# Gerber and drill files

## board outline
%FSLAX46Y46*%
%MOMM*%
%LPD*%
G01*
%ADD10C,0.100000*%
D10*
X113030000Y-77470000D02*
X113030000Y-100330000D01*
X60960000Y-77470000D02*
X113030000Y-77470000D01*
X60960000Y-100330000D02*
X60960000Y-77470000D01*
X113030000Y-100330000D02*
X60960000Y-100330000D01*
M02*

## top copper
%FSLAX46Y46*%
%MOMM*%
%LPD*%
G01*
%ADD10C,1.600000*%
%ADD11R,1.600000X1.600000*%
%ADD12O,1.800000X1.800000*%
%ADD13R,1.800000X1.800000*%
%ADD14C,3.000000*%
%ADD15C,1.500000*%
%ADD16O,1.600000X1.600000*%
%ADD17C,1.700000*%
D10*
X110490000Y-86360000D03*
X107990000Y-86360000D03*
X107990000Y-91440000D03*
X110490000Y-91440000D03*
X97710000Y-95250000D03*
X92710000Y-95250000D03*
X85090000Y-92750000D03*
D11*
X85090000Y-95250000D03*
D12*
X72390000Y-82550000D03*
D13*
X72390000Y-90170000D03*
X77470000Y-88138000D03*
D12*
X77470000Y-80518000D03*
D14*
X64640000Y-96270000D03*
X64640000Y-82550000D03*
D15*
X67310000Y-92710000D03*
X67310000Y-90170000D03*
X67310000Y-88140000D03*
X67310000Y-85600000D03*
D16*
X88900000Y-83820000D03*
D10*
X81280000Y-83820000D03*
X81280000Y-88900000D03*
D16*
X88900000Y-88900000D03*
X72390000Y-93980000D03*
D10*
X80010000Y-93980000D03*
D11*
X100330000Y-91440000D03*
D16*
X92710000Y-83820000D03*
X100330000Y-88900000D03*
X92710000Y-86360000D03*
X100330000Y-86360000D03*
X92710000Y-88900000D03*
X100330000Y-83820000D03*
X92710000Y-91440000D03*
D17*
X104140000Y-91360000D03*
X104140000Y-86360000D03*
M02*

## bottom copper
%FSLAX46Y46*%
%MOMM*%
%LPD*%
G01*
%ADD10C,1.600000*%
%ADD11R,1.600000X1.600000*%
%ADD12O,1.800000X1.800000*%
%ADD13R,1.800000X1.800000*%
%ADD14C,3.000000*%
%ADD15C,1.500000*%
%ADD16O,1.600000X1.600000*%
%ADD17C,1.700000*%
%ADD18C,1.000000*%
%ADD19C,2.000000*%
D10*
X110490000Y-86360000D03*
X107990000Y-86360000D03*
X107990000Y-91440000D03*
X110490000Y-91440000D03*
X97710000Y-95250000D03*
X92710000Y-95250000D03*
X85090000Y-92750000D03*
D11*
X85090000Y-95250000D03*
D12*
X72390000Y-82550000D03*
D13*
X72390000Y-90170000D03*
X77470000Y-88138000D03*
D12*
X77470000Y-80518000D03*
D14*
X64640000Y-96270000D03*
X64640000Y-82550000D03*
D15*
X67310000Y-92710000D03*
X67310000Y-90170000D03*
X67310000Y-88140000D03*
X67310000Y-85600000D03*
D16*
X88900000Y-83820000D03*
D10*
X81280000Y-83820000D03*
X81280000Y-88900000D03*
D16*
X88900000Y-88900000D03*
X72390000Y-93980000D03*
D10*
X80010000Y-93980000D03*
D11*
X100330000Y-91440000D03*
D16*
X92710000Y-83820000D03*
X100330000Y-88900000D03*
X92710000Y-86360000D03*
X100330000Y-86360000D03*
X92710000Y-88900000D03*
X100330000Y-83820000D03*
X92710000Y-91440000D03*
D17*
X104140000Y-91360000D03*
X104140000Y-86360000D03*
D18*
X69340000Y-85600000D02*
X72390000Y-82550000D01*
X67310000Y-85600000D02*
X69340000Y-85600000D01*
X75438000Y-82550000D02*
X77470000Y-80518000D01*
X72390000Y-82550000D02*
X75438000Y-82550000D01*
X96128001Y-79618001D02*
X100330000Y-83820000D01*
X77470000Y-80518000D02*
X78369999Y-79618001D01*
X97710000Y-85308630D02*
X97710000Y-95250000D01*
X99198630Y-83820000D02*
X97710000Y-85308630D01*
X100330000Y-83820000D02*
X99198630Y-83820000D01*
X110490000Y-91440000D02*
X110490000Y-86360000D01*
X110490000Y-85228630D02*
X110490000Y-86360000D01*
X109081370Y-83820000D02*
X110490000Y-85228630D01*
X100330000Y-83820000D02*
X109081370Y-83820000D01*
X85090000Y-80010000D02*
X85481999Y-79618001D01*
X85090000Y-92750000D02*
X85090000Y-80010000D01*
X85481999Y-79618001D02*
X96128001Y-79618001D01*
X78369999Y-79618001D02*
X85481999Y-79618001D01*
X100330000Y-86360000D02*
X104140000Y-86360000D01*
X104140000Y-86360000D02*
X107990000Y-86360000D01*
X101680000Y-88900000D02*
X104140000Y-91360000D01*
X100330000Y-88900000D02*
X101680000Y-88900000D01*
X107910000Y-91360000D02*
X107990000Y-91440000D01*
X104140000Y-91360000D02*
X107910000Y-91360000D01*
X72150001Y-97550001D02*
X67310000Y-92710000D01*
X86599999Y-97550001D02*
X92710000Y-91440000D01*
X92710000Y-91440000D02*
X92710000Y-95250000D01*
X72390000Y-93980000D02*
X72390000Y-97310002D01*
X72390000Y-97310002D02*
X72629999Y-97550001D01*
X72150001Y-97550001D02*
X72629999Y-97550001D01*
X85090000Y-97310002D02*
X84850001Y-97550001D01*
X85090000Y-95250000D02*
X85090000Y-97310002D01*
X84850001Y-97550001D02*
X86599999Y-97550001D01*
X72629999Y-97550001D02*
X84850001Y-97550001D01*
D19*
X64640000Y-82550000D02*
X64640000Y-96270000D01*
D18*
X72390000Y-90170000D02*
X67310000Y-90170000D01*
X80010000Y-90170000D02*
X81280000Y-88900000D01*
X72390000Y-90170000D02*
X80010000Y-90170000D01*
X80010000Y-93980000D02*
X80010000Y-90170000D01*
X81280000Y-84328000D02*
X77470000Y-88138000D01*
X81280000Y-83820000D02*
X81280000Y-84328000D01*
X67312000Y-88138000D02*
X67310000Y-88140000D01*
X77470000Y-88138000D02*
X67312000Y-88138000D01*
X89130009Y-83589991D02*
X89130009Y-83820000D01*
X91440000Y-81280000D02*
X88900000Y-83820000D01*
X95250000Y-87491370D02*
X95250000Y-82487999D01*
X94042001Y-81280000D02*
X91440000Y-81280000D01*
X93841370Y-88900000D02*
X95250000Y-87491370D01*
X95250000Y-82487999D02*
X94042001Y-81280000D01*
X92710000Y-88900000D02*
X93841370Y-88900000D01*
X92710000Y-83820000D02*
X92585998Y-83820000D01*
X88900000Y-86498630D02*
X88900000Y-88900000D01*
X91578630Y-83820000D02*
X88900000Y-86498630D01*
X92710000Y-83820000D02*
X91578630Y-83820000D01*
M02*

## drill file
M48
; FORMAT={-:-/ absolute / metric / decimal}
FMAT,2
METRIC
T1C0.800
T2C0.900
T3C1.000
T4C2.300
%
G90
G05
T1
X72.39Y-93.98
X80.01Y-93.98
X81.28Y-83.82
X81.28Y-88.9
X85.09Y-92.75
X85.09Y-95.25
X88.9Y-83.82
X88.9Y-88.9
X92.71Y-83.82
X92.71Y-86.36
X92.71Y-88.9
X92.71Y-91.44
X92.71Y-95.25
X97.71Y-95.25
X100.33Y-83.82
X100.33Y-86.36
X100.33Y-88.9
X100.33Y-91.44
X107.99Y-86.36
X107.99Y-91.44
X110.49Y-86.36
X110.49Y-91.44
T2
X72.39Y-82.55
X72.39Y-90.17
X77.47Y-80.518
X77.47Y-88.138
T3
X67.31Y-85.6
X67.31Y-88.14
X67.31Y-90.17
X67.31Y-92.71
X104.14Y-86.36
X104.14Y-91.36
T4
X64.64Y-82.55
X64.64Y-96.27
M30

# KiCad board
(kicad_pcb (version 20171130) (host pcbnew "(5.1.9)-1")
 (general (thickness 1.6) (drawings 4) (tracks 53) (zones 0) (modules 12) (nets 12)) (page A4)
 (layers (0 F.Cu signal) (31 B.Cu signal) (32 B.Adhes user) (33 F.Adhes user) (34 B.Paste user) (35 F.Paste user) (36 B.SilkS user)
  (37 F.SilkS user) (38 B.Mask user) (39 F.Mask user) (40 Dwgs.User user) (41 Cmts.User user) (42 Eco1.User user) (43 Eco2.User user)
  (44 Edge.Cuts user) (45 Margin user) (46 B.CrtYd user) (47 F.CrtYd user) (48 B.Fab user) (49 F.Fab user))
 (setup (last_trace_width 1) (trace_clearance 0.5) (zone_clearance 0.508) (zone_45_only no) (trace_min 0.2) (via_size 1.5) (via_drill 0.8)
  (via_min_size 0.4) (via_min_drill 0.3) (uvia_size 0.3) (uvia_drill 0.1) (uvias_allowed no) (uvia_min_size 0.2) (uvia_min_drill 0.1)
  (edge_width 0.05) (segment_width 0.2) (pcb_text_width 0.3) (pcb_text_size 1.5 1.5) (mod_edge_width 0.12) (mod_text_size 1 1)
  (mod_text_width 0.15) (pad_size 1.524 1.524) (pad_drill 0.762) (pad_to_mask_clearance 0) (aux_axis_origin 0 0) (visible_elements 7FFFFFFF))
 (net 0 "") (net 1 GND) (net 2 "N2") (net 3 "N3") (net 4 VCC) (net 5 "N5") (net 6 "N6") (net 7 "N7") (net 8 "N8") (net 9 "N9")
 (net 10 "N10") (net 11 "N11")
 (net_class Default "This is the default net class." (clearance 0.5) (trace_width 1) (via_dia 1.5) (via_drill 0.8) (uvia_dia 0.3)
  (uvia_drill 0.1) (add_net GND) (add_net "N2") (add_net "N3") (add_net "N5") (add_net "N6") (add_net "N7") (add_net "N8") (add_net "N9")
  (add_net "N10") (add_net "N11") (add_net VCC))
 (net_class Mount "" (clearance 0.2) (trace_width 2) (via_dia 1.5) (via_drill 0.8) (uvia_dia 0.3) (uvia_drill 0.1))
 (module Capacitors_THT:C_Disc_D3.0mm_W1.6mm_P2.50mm (layer F.Cu) (at 110.49 86.36 180)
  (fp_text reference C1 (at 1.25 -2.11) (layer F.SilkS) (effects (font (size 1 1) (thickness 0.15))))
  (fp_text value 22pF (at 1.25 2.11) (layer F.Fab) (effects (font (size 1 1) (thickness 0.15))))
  (pad 1 thru_hole circle (at 0 0 180) (size 1.6 1.6) (drill 0.8) (layers *.Cu *.Mask) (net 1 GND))
  (pad 2 thru_hole circle (at 2.5 0 180) (size 1.6 1.6) (drill 0.8) (layers *.Cu *.Mask) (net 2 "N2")))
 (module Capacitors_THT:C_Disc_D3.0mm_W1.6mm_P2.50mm (layer F.Cu) (at 110.49 91.44 180)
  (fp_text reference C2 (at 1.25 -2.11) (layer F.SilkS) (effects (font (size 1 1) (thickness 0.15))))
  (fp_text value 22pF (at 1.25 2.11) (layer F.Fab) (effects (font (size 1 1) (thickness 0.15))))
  (pad 2 thru_hole circle (at 2.5 0 180) (size 1.6 1.6) (drill 0.8) (layers *.Cu *.Mask) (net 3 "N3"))
  (pad 1 thru_hole circle (at 0 0 180) (size 1.6 1.6) (drill 0.8) (layers *.Cu *.Mask) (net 1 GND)))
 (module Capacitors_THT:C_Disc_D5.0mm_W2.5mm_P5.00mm (layer F.Cu) (at 92.71 95.25)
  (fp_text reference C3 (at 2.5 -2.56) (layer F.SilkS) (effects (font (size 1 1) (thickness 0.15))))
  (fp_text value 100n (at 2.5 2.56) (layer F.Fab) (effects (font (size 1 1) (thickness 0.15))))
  (pad 2 thru_hole circle (at 5 0) (size 1.6 1.6) (drill 0.8) (layers *.Cu *.Mask) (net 1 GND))
  (pad 1 thru_hole circle (at 0 0) (size 1.6 1.6) (drill 0.8) (layers *.Cu *.Mask) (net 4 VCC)))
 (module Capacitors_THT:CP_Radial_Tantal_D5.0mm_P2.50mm (layer F.Cu) (at 85.09 95.25 90)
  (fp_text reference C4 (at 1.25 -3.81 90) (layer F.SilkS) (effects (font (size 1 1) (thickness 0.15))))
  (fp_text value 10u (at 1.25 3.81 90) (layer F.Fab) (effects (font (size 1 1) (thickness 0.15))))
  (pad 2 thru_hole circle (at 2.5 0 90) (size 1.6 1.6) (drill 0.8) (layers *.Cu *.Mask) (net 1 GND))
  (pad 1 thru_hole rect (at 0 0 90) (size 1.6 1.6) (drill 0.8) (layers *.Cu *.Mask) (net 4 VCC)))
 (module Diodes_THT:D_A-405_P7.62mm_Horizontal (layer F.Cu) (at 72.39 90.17 90)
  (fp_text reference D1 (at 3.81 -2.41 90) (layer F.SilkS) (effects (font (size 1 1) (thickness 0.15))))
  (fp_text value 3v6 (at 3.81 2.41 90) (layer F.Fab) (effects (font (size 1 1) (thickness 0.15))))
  (pad 2 thru_hole oval (at 7.62 0 90) (size 1.8 1.8) (drill 0.9) (layers *.Cu *.Mask) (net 1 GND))
  (pad 1 thru_hole rect (at 0 0 90) (size 1.8 1.8) (drill 0.9) (layers *.Cu *.Mask) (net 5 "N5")))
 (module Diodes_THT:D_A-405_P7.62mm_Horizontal (layer F.Cu) (at 77.47 88.138 90)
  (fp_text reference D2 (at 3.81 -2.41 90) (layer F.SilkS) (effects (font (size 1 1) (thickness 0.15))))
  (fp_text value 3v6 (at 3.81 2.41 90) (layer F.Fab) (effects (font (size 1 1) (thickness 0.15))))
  (pad 1 thru_hole rect (at 0 0 90) (size 1.8 1.8) (drill 0.9) (layers *.Cu *.Mask) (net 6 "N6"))
  (pad 2 thru_hole oval (at 7.62 0 90) (size 1.8 1.8) (drill 0.9) (layers *.Cu *.Mask) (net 1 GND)))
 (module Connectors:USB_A (layer B.Cu) (at 67.31 92.71 90)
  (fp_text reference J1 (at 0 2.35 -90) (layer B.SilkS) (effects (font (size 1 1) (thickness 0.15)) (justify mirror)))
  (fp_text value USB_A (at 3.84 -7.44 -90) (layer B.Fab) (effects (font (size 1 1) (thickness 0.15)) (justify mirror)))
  (pad 5 thru_hole circle (at -3.56 -2.67 180) (size 3 3) (drill 2.3) (layers *.Cu *.Mask) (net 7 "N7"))
  (pad 5 thru_hole circle (at 10.16 -2.67 180) (size 3 3) (drill 2.3) (layers *.Cu *.Mask) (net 7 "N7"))
  (pad 1 thru_hole circle (at 0 0 180) (size 1.5 1.5) (drill 1) (layers *.Cu *.Mask) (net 4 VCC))
  (pad 2 thru_hole circle (at 2.54 0 180) (size 1.5 1.5) (drill 1) (layers *.Cu *.Mask) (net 5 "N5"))
  (pad 3 thru_hole circle (at 4.57 0 180) (size 1.5 1.5) (drill 1) (layers *.Cu *.Mask) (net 6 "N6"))
  (pad 4 thru_hole circle (at 7.11 0 180) (size 1.5 1.5) (drill 1) (layers *.Cu *.Mask) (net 1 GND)))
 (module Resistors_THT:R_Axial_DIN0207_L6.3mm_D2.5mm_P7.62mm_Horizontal (layer F.Cu) (at 81.28 83.82)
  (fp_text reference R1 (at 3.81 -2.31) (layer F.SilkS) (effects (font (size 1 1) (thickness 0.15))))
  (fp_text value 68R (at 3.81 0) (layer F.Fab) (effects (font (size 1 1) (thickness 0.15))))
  (pad 2 thru_hole oval (at 7.62 0) (size 1.6 1.6) (drill 0.8) (layers *.Cu *.Mask) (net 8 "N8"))
  (pad 1 thru_hole circle (at 0 0) (size 1.6 1.6) (drill 0.8) (layers *.Cu *.Mask) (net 6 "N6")))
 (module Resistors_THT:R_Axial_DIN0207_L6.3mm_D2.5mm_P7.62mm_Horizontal (layer F.Cu) (at 81.28 88.9)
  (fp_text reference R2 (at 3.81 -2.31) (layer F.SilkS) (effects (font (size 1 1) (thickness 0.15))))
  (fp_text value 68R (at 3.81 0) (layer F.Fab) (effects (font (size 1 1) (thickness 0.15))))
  (pad 1 thru_hole circle (at 0 0) (size 1.6 1.6) (drill 0.8) (layers *.Cu *.Mask) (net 5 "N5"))
  (pad 2 thru_hole oval (at 7.62 0) (size 1.6 1.6) (drill 0.8) (layers *.Cu *.Mask) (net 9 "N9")))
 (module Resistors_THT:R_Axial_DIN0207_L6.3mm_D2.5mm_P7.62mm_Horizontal (layer F.Cu) (at 80.01 93.98 180)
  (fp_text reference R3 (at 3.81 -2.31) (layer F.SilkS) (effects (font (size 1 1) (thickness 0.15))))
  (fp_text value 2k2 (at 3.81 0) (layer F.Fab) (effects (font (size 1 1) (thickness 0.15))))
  (pad 2 thru_hole oval (at 7.62 0 180) (size 1.6 1.6) (drill 0.8) (layers *.Cu *.Mask) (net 4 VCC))
  (pad 1 thru_hole circle (at 0 0 180) (size 1.6 1.6) (drill 0.8) (layers *.Cu *.Mask) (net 5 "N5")))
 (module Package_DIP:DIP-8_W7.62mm (layer F.Cu) (at 100.33 91.44 180)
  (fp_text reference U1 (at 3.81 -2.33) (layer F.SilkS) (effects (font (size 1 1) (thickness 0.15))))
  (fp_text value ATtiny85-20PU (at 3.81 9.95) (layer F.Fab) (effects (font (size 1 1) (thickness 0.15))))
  (pad 1 thru_hole rect (at 0 0 180) (size 1.6 1.6) (drill 0.8) (layers *.Cu *.Mask) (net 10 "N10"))
  (pad 5 thru_hole oval (at 7.62 7.62 180) (size 1.6 1.6) (drill 0.8) (layers *.Cu *.Mask) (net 9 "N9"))
  (pad 2 thru_hole oval (at 0 2.54 180) (size 1.6 1.6) (drill 0.8) (layers *.Cu *.Mask) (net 3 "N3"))
  (pad 6 thru_hole oval (at 7.62 5.08 180) (size 1.6 1.6) (drill 0.8) (layers *.Cu *.Mask) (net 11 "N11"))
  (pad 3 thru_hole oval (at 0 5.08 180) (size 1.6 1.6) (drill 0.8) (layers *.Cu *.Mask) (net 2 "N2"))
  (pad 7 thru_hole oval (at 7.62 2.54 180) (size 1.6 1.6) (drill 0.8) (layers *.Cu *.Mask) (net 8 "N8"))
  (pad 4 thru_hole oval (at 0 7.62 180) (size 1.6 1.6) (drill 0.8) (layers *.Cu *.Mask) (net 1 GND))
  (pad 8 thru_hole oval (at 7.62 0 180) (size 1.6 1.6) (drill 0.8) (layers *.Cu *.Mask) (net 4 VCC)))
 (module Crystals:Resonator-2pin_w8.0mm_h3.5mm (layer F.Cu) (at 104.14 86.36 270)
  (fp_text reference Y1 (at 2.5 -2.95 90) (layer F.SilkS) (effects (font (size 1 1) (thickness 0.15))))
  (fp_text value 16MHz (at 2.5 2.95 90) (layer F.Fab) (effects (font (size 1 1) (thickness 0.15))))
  (pad 2 thru_hole circle (at 5 0 270) (size 1.7 1.7) (drill 1) (layers *.Cu *.Mask) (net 3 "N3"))
  (pad 1 thru_hole circle (at 0 0 270) (size 1.7 1.7) (drill 1) (layers *.Cu *.Mask) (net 2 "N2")))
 (gr_line (start 113.03 77.47) (end 113.03 100.33) (layer Edge.Cuts) (width 0.1))
 (gr_line (start 60.96 77.47) (end 113.03 77.47) (layer Edge.Cuts) (width 0.1))
 (gr_line (start 60.96 100.33) (end 60.96 77.47) (layer Edge.Cuts) (width 0.1))
 (gr_line (start 113.03 100.33) (end 60.96 100.33) (layer Edge.Cuts) (width 0.1))
 (segment (start 69.34 85.6) (end 72.39 82.55) (width 1) (layer B.Cu) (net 1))
 (segment (start 67.31 85.6) (end 69.34 85.6) (width 1) (layer B.Cu) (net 1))
 (segment (start 75.438 82.55) (end 77.47 80.518) (width 1) (layer B.Cu) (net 1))
 (segment (start 72.39 82.55) (end 75.438 82.55) (width 1) (layer B.Cu) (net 1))
 (segment (start 96.128001 79.618001) (end 100.33 83.82) (width 1) (layer B.Cu) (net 1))
 (segment (start 77.47 80.518) (end 78.369999 79.618001) (width 1) (layer B.Cu) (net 1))
 (segment (start 97.71 85.30863) (end 97.71 95.25) (width 1) (layer B.Cu) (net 1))
 (segment (start 99.19863 83.82) (end 97.71 85.30863) (width 1) (layer B.Cu) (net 1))
 (segment (start 100.33 83.82) (end 99.19863 83.82) (width 1) (layer B.Cu) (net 1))
 (segment (start 110.49 91.44) (end 110.49 86.36) (width 1) (layer B.Cu) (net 1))
 (segment (start 110.49 85.22863) (end 110.49 86.36) (width 1) (layer B.Cu) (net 1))
 (segment (start 109.08137 83.82) (end 110.49 85.22863) (width 1) (layer B.Cu) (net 1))
 (segment (start 100.33 83.82) (end 109.08137 83.82) (width 1) (layer B.Cu) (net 1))
 (segment (start 85.09 80.01) (end 85.481999 79.618001) (width 1) (layer B.Cu) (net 1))
 (segment (start 85.09 92.75) (end 85.09 80.01) (width 1) (layer B.Cu) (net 1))
 (segment (start 85.481999 79.618001) (end 96.128001 79.618001) (width 1) (layer B.Cu) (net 1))
 (segment (start 78.369999 79.618001) (end 85.481999 79.618001) (width 1) (layer B.Cu) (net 1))
 (segment (start 100.33 86.36) (end 104.14 86.36) (width 1) (layer B.Cu) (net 2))
 (segment (start 104.14 86.36) (end 107.99 86.36) (width 1) (layer B.Cu) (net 2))
 (segment (start 101.68 88.9) (end 104.14 91.36) (width 1) (layer B.Cu) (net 3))
 (segment (start 100.33 88.9) (end 101.68 88.9) (width 1) (layer B.Cu) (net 3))
 (segment (start 107.91 91.36) (end 107.99 91.44) (width 1) (layer B.Cu) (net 3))
 (segment (start 104.14 91.36) (end 107.91 91.36) (width 1) (layer B.Cu) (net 3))
 (segment (start 72.150001 97.550001) (end 67.31 92.71) (width 1) (layer B.Cu) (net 4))
 (segment (start 86.599999 97.550001) (end 92.71 91.44) (width 1) (layer B.Cu) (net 4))
 (segment (start 92.71 91.44) (end 92.71 95.25) (width 1) (layer B.Cu) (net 4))
 (segment (start 72.39 93.98) (end 72.39 97.310002) (width 1) (layer B.Cu) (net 4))
 (segment (start 72.39 97.310002) (end 72.629999 97.550001) (width 1) (layer B.Cu) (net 4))
 (segment (start 72.150001 97.550001) (end 72.629999 97.550001) (width 1) (layer B.Cu) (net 4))
 (segment (start 85.09 97.310002) (end 84.850001 97.550001) (width 1) (layer B.Cu) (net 4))
 (segment (start 85.09 95.25) (end 85.09 97.310002) (width 1) (layer B.Cu) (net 4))
 (segment (start 84.850001 97.550001) (end 86.599999 97.550001) (width 1) (layer B.Cu) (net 4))
 (segment (start 72.629999 97.550001) (end 84.850001 97.550001) (width 1) (layer B.Cu) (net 4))
 (segment (start 64.64 82.55) (end 64.64 96.27) (width 2) (layer B.Cu) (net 7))
 (segment (start 72.39 90.17) (end 67.31 90.17) (width 1) (layer B.Cu) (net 5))
 (segment (start 80.01 90.17) (end 81.28 88.9) (width 1) (layer B.Cu) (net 5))
 (segment (start 72.39 90.17) (end 80.01 90.17) (width 1) (layer B.Cu) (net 5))
 (segment (start 80.01 93.98) (end 80.01 90.17) (width 1) (layer B.Cu) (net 5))
 (segment (start 81.28 84.328) (end 77.47 88.138) (width 1) (layer B.Cu) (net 6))
 (segment (start 81.28 83.82) (end 81.28 84.328) (width 1) (layer B.Cu) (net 6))
 (segment (start 67.312 88.138) (end 67.31 88.14) (width 1) (layer B.Cu) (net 6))
 (segment (start 77.47 88.138) (end 67.312 88.138) (width 1) (layer B.Cu) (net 6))
 (segment (start 89.130009 83.589991) (end 89.130009 83.82) (width 1) (layer B.Cu) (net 8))
 (segment (start 91.44 81.28) (end 88.9 83.82) (width 1) (layer B.Cu) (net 8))
 (segment (start 95.25 87.49137) (end 95.25 82.487999) (width 1) (layer B.Cu) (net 8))
 (segment (start 94.042001 81.28) (end 91.44 81.28) (width 1) (layer B.Cu) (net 8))
 (segment (start 93.84137 88.9) (end 95.25 87.49137) (width 1) (layer B.Cu) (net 8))
 (segment (start 95.25 82.487999) (end 94.042001 81.28) (width 1) (layer B.Cu) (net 8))
 (segment (start 92.71 88.9) (end 93.84137 88.9) (width 1) (layer B.Cu) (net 8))
 (segment (start 92.71 83.82) (end 92.585998 83.82) (width 1) (layer B.Cu) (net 9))
 (segment (start 88.9 86.49863) (end 88.9 88.9) (width 1) (layer B.Cu) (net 9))
 (segment (start 91.57863 83.82) (end 88.9 86.49863) (width 1) (layer B.Cu) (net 9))
 (segment (start 92.71 83.82) (end 91.57863 83.82) (width 1) (layer B.Cu) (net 9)))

